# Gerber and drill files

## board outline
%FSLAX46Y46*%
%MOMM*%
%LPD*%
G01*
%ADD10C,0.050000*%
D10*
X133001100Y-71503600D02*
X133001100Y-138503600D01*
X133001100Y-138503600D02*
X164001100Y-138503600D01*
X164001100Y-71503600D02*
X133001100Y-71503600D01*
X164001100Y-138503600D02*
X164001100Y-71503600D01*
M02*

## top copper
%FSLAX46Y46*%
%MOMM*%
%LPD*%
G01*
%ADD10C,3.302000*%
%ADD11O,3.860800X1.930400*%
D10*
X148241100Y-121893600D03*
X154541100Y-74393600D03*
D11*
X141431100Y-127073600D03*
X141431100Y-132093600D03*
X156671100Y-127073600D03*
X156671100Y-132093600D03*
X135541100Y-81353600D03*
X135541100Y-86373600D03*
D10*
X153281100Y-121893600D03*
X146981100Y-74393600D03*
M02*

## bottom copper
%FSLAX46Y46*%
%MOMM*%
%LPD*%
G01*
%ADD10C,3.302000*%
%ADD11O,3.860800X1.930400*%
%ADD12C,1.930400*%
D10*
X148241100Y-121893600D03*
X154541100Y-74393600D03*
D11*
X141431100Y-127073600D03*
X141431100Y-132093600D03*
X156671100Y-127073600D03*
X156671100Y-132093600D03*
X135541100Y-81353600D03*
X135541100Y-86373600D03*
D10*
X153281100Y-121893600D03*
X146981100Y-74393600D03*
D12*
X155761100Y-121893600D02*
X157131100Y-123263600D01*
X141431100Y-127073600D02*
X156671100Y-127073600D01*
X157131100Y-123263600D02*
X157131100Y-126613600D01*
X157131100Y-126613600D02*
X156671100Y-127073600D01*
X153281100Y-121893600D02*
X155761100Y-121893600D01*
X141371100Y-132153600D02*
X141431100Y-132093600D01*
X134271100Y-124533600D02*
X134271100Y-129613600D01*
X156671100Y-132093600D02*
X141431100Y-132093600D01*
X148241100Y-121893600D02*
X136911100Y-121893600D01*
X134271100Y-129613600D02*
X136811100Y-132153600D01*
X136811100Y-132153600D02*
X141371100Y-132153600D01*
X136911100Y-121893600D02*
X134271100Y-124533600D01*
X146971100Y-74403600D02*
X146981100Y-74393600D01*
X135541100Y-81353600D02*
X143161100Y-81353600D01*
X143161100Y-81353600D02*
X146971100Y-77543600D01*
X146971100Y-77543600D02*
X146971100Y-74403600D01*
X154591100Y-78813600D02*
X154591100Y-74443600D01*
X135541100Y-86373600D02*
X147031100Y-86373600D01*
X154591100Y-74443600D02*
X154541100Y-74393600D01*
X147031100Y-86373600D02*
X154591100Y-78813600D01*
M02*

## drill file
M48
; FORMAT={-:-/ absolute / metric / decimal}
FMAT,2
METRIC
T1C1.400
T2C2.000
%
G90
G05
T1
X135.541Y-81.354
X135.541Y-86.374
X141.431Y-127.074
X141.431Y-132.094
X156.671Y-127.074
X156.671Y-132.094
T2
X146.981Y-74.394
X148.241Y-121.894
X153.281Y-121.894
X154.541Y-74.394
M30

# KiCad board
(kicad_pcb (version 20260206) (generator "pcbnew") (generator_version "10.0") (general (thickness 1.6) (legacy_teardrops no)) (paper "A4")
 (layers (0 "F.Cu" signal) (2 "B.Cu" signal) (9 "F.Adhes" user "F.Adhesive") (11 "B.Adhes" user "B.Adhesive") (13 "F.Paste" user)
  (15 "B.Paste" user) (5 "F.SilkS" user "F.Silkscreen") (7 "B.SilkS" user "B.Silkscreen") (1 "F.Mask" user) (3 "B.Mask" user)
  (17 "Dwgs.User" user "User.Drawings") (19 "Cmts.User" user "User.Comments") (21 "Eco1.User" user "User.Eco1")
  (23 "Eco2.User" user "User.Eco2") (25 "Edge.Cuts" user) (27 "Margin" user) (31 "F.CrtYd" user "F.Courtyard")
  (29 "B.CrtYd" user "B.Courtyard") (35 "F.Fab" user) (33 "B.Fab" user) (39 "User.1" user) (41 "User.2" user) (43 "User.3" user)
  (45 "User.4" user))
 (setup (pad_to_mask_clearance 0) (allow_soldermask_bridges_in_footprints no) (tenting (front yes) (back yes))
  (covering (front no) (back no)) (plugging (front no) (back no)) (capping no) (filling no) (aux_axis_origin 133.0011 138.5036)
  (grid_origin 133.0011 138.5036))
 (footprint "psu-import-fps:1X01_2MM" (layer "F.Cu") (at 148.2411 121.8936)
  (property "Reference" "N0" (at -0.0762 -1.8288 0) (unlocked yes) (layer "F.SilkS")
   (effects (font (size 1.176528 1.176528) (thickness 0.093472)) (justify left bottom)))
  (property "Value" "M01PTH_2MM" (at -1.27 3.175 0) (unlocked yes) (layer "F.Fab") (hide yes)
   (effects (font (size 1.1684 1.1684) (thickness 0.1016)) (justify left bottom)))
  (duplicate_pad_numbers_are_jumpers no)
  (pad "1" thru_hole circle (at 0 0 90) (size 3.302 3.302) (drill 2) (layers "*.Cu" "*.Mask") (remove_unused_layers no) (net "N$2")
   (solder_mask_margin 0.1016) (thermal_bridge_angle 0)))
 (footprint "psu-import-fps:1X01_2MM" (layer "F.Cu") (at 154.5411 74.3936)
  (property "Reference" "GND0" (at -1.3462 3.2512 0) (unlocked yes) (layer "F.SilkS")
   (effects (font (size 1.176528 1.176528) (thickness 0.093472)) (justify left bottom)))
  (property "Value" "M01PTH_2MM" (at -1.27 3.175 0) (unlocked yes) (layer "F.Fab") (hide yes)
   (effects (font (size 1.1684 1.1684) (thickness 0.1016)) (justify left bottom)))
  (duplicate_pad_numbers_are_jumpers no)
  (pad "1" thru_hole circle (at 0 0 90) (size 3.302 3.302) (drill 2) (layers "*.Cu" "*.Mask") (remove_unused_layers no) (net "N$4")
   (solder_mask_margin 0.1016) (thermal_bridge_angle 0)))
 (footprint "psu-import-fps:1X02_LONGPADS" (layer "F.Cu") (at 141.4311 127.0736 -90)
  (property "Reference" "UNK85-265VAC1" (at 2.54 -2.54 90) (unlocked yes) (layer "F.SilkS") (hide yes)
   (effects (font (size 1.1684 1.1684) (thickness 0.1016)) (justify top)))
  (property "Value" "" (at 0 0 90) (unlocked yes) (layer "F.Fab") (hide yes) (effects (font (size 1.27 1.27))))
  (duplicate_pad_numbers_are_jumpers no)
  (pad "1" thru_hole oval (at 0 0) (size 3.8608 1.9304) (drill 1.4) (layers "*.Cu" "*.Mask") (remove_unused_layers no) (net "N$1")
   (solder_mask_margin 0.1016) (thermal_bridge_angle 0))
  (pad "2" thru_hole oval (at 5.02 0) (size 3.8608 1.9304) (drill 1.4) (layers "*.Cu" "*.Mask") (remove_unused_layers no) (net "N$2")
   (solder_mask_margin 0.1016) (thermal_bridge_angle 0)))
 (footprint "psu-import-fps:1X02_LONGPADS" (layer "F.Cu") (at 156.6711 127.0736 -90)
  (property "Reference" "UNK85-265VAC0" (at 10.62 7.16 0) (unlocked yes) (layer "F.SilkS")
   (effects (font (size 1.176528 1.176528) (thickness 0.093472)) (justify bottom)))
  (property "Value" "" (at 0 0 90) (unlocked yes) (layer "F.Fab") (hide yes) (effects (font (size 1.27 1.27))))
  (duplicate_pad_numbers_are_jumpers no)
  (pad "1" thru_hole oval (at 0 0) (size 3.8608 1.9304) (drill 1.4) (layers "*.Cu" "*.Mask") (remove_unused_layers no) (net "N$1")
   (solder_mask_margin 0.1016) (thermal_bridge_angle 0))
  (pad "2" thru_hole oval (at 5.02 0) (size 3.8608 1.9304) (drill 1.4) (layers "*.Cu" "*.Mask") (remove_unused_layers no) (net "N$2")
   (solder_mask_margin 0.1016) (thermal_bridge_angle 0)))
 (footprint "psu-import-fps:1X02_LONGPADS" (layer "F.Cu") (at 135.5411 81.3536 -90)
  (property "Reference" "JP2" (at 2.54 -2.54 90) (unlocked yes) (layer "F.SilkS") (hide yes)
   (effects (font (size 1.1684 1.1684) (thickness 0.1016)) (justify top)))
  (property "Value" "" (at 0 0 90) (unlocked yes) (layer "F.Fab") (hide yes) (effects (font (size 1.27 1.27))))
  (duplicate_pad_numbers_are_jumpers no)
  (pad "1" thru_hole oval (at 0 0) (size 3.8608 1.9304) (drill 1.4) (layers "*.Cu" "*.Mask") (remove_unused_layers no) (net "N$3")
   (solder_mask_margin 0.1016) (thermal_bridge_angle 0))
  (pad "2" thru_hole oval (at 5.02 0) (size 3.8608 1.9304) (drill 1.4) (layers "*.Cu" "*.Mask") (remove_unused_layers no) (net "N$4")
   (solder_mask_margin 0.1016) (thermal_bridge_angle 0)))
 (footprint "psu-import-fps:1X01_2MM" (layer "F.Cu") (at 153.2811 121.8936)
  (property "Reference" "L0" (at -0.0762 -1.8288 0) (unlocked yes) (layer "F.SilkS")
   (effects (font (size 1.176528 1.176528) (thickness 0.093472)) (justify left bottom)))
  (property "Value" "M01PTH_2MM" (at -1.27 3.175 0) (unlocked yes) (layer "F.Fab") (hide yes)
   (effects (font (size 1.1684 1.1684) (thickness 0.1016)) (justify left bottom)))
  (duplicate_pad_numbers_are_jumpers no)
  (pad "1" thru_hole circle (at 0 0 90) (size 3.302 3.302) (drill 2) (layers "*.Cu" "*.Mask") (remove_unused_layers no) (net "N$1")
   (solder_mask_margin 0.1016) (thermal_bridge_angle 0)))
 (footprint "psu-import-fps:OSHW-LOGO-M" (layer "F.Cu") (at 135.5411 75.0036 90)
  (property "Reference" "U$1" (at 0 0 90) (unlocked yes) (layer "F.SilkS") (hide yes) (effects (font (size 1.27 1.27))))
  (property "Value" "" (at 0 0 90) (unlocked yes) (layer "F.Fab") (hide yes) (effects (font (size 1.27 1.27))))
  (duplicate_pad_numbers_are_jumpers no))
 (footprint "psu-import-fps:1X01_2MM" (layer "F.Cu") (at 146.9811 74.3936)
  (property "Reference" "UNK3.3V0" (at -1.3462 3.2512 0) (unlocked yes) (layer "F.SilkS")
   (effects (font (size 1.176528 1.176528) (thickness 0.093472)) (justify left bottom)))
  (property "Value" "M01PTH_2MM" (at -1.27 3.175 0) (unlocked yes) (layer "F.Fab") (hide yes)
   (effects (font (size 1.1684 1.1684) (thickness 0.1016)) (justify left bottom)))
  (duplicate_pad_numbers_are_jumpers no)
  (pad "1" thru_hole circle (at 0 0 90) (size 3.302 3.302) (drill 2) (layers "*.Cu" "*.Mask") (remove_unused_layers no) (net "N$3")
   (solder_mask_margin 0.1016) (thermal_bridge_angle 0)))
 (gr_line (start 133.0011 71.5036) (end 133.0011 138.5036) (stroke (width 0.05) (type solid)) (layer "Edge.Cuts"))
 (gr_line (start 133.0011 138.5036) (end 164.0011 138.5036) (stroke (width 0.05) (type solid)) (layer "Edge.Cuts"))
 (gr_line (start 164.0011 71.5036) (end 133.0011 71.5036) (stroke (width 0.05) (type solid)) (layer "Edge.Cuts"))
 (gr_line (start 164.0011 138.5036) (end 164.0011 71.5036) (stroke (width 0.05) (type solid)) (layer "Edge.Cuts"))
 (segment (start 155.7611 121.8936) (end 157.1311 123.2636) (width 1.9304) (layer "B.Cu") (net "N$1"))
 (segment (start 141.4311 127.0736) (end 156.6711 127.0736) (width 1.9304) (layer "B.Cu") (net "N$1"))
 (segment (start 157.1311 123.2636) (end 157.1311 126.6136) (width 1.9304) (layer "B.Cu") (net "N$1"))
 (segment (start 157.1311 126.6136) (end 156.6711 127.0736) (width 1.9304) (layer "B.Cu") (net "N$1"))
 (segment (start 153.2811 121.8936) (end 155.7611 121.8936) (width 1.9304) (layer "B.Cu") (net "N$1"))
 (segment (start 141.3711 132.1536) (end 141.4311 132.0936) (width 1.9304) (layer "B.Cu") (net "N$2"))
 (segment (start 134.2711 124.5336) (end 134.2711 129.6136) (width 1.9304) (layer "B.Cu") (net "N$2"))
 (segment (start 156.6711 132.0936) (end 141.4311 132.0936) (width 1.9304) (layer "B.Cu") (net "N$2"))
 (segment (start 148.2411 121.8936) (end 136.9111 121.8936) (width 1.9304) (layer "B.Cu") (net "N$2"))
 (segment (start 134.2711 129.6136) (end 136.8111 132.1536) (width 1.9304) (layer "B.Cu") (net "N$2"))
 (segment (start 136.8111 132.1536) (end 141.3711 132.1536) (width 1.9304) (layer "B.Cu") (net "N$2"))
 (segment (start 136.9111 121.8936) (end 134.2711 124.5336) (width 1.9304) (layer "B.Cu") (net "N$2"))
 (segment (start 146.9711 74.4036) (end 146.9811 74.3936) (width 1.9304) (layer "B.Cu") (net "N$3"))
 (segment (start 135.5411 81.3536) (end 143.1611 81.3536) (width 1.9304) (layer "B.Cu") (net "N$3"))
 (segment (start 143.1611 81.3536) (end 146.9711 77.5436) (width 1.9304) (layer "B.Cu") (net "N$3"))
 (segment (start 146.9711 77.5436) (end 146.9711 74.4036) (width 1.9304) (layer "B.Cu") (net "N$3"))
 (segment (start 154.5911 78.8136) (end 154.5911 74.4436) (width 1.9304) (layer "B.Cu") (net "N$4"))
 (segment (start 135.5411 86.3736) (end 147.0311 86.3736) (width 1.9304) (layer "B.Cu") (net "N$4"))
 (segment (start 154.5911 74.4436) (end 154.5411 74.3936) (width 1.9304) (layer "B.Cu") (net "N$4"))
 (segment (start 147.0311 86.3736) (end 154.5911 78.8136) (width 1.9304) (layer "B.Cu") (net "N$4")))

